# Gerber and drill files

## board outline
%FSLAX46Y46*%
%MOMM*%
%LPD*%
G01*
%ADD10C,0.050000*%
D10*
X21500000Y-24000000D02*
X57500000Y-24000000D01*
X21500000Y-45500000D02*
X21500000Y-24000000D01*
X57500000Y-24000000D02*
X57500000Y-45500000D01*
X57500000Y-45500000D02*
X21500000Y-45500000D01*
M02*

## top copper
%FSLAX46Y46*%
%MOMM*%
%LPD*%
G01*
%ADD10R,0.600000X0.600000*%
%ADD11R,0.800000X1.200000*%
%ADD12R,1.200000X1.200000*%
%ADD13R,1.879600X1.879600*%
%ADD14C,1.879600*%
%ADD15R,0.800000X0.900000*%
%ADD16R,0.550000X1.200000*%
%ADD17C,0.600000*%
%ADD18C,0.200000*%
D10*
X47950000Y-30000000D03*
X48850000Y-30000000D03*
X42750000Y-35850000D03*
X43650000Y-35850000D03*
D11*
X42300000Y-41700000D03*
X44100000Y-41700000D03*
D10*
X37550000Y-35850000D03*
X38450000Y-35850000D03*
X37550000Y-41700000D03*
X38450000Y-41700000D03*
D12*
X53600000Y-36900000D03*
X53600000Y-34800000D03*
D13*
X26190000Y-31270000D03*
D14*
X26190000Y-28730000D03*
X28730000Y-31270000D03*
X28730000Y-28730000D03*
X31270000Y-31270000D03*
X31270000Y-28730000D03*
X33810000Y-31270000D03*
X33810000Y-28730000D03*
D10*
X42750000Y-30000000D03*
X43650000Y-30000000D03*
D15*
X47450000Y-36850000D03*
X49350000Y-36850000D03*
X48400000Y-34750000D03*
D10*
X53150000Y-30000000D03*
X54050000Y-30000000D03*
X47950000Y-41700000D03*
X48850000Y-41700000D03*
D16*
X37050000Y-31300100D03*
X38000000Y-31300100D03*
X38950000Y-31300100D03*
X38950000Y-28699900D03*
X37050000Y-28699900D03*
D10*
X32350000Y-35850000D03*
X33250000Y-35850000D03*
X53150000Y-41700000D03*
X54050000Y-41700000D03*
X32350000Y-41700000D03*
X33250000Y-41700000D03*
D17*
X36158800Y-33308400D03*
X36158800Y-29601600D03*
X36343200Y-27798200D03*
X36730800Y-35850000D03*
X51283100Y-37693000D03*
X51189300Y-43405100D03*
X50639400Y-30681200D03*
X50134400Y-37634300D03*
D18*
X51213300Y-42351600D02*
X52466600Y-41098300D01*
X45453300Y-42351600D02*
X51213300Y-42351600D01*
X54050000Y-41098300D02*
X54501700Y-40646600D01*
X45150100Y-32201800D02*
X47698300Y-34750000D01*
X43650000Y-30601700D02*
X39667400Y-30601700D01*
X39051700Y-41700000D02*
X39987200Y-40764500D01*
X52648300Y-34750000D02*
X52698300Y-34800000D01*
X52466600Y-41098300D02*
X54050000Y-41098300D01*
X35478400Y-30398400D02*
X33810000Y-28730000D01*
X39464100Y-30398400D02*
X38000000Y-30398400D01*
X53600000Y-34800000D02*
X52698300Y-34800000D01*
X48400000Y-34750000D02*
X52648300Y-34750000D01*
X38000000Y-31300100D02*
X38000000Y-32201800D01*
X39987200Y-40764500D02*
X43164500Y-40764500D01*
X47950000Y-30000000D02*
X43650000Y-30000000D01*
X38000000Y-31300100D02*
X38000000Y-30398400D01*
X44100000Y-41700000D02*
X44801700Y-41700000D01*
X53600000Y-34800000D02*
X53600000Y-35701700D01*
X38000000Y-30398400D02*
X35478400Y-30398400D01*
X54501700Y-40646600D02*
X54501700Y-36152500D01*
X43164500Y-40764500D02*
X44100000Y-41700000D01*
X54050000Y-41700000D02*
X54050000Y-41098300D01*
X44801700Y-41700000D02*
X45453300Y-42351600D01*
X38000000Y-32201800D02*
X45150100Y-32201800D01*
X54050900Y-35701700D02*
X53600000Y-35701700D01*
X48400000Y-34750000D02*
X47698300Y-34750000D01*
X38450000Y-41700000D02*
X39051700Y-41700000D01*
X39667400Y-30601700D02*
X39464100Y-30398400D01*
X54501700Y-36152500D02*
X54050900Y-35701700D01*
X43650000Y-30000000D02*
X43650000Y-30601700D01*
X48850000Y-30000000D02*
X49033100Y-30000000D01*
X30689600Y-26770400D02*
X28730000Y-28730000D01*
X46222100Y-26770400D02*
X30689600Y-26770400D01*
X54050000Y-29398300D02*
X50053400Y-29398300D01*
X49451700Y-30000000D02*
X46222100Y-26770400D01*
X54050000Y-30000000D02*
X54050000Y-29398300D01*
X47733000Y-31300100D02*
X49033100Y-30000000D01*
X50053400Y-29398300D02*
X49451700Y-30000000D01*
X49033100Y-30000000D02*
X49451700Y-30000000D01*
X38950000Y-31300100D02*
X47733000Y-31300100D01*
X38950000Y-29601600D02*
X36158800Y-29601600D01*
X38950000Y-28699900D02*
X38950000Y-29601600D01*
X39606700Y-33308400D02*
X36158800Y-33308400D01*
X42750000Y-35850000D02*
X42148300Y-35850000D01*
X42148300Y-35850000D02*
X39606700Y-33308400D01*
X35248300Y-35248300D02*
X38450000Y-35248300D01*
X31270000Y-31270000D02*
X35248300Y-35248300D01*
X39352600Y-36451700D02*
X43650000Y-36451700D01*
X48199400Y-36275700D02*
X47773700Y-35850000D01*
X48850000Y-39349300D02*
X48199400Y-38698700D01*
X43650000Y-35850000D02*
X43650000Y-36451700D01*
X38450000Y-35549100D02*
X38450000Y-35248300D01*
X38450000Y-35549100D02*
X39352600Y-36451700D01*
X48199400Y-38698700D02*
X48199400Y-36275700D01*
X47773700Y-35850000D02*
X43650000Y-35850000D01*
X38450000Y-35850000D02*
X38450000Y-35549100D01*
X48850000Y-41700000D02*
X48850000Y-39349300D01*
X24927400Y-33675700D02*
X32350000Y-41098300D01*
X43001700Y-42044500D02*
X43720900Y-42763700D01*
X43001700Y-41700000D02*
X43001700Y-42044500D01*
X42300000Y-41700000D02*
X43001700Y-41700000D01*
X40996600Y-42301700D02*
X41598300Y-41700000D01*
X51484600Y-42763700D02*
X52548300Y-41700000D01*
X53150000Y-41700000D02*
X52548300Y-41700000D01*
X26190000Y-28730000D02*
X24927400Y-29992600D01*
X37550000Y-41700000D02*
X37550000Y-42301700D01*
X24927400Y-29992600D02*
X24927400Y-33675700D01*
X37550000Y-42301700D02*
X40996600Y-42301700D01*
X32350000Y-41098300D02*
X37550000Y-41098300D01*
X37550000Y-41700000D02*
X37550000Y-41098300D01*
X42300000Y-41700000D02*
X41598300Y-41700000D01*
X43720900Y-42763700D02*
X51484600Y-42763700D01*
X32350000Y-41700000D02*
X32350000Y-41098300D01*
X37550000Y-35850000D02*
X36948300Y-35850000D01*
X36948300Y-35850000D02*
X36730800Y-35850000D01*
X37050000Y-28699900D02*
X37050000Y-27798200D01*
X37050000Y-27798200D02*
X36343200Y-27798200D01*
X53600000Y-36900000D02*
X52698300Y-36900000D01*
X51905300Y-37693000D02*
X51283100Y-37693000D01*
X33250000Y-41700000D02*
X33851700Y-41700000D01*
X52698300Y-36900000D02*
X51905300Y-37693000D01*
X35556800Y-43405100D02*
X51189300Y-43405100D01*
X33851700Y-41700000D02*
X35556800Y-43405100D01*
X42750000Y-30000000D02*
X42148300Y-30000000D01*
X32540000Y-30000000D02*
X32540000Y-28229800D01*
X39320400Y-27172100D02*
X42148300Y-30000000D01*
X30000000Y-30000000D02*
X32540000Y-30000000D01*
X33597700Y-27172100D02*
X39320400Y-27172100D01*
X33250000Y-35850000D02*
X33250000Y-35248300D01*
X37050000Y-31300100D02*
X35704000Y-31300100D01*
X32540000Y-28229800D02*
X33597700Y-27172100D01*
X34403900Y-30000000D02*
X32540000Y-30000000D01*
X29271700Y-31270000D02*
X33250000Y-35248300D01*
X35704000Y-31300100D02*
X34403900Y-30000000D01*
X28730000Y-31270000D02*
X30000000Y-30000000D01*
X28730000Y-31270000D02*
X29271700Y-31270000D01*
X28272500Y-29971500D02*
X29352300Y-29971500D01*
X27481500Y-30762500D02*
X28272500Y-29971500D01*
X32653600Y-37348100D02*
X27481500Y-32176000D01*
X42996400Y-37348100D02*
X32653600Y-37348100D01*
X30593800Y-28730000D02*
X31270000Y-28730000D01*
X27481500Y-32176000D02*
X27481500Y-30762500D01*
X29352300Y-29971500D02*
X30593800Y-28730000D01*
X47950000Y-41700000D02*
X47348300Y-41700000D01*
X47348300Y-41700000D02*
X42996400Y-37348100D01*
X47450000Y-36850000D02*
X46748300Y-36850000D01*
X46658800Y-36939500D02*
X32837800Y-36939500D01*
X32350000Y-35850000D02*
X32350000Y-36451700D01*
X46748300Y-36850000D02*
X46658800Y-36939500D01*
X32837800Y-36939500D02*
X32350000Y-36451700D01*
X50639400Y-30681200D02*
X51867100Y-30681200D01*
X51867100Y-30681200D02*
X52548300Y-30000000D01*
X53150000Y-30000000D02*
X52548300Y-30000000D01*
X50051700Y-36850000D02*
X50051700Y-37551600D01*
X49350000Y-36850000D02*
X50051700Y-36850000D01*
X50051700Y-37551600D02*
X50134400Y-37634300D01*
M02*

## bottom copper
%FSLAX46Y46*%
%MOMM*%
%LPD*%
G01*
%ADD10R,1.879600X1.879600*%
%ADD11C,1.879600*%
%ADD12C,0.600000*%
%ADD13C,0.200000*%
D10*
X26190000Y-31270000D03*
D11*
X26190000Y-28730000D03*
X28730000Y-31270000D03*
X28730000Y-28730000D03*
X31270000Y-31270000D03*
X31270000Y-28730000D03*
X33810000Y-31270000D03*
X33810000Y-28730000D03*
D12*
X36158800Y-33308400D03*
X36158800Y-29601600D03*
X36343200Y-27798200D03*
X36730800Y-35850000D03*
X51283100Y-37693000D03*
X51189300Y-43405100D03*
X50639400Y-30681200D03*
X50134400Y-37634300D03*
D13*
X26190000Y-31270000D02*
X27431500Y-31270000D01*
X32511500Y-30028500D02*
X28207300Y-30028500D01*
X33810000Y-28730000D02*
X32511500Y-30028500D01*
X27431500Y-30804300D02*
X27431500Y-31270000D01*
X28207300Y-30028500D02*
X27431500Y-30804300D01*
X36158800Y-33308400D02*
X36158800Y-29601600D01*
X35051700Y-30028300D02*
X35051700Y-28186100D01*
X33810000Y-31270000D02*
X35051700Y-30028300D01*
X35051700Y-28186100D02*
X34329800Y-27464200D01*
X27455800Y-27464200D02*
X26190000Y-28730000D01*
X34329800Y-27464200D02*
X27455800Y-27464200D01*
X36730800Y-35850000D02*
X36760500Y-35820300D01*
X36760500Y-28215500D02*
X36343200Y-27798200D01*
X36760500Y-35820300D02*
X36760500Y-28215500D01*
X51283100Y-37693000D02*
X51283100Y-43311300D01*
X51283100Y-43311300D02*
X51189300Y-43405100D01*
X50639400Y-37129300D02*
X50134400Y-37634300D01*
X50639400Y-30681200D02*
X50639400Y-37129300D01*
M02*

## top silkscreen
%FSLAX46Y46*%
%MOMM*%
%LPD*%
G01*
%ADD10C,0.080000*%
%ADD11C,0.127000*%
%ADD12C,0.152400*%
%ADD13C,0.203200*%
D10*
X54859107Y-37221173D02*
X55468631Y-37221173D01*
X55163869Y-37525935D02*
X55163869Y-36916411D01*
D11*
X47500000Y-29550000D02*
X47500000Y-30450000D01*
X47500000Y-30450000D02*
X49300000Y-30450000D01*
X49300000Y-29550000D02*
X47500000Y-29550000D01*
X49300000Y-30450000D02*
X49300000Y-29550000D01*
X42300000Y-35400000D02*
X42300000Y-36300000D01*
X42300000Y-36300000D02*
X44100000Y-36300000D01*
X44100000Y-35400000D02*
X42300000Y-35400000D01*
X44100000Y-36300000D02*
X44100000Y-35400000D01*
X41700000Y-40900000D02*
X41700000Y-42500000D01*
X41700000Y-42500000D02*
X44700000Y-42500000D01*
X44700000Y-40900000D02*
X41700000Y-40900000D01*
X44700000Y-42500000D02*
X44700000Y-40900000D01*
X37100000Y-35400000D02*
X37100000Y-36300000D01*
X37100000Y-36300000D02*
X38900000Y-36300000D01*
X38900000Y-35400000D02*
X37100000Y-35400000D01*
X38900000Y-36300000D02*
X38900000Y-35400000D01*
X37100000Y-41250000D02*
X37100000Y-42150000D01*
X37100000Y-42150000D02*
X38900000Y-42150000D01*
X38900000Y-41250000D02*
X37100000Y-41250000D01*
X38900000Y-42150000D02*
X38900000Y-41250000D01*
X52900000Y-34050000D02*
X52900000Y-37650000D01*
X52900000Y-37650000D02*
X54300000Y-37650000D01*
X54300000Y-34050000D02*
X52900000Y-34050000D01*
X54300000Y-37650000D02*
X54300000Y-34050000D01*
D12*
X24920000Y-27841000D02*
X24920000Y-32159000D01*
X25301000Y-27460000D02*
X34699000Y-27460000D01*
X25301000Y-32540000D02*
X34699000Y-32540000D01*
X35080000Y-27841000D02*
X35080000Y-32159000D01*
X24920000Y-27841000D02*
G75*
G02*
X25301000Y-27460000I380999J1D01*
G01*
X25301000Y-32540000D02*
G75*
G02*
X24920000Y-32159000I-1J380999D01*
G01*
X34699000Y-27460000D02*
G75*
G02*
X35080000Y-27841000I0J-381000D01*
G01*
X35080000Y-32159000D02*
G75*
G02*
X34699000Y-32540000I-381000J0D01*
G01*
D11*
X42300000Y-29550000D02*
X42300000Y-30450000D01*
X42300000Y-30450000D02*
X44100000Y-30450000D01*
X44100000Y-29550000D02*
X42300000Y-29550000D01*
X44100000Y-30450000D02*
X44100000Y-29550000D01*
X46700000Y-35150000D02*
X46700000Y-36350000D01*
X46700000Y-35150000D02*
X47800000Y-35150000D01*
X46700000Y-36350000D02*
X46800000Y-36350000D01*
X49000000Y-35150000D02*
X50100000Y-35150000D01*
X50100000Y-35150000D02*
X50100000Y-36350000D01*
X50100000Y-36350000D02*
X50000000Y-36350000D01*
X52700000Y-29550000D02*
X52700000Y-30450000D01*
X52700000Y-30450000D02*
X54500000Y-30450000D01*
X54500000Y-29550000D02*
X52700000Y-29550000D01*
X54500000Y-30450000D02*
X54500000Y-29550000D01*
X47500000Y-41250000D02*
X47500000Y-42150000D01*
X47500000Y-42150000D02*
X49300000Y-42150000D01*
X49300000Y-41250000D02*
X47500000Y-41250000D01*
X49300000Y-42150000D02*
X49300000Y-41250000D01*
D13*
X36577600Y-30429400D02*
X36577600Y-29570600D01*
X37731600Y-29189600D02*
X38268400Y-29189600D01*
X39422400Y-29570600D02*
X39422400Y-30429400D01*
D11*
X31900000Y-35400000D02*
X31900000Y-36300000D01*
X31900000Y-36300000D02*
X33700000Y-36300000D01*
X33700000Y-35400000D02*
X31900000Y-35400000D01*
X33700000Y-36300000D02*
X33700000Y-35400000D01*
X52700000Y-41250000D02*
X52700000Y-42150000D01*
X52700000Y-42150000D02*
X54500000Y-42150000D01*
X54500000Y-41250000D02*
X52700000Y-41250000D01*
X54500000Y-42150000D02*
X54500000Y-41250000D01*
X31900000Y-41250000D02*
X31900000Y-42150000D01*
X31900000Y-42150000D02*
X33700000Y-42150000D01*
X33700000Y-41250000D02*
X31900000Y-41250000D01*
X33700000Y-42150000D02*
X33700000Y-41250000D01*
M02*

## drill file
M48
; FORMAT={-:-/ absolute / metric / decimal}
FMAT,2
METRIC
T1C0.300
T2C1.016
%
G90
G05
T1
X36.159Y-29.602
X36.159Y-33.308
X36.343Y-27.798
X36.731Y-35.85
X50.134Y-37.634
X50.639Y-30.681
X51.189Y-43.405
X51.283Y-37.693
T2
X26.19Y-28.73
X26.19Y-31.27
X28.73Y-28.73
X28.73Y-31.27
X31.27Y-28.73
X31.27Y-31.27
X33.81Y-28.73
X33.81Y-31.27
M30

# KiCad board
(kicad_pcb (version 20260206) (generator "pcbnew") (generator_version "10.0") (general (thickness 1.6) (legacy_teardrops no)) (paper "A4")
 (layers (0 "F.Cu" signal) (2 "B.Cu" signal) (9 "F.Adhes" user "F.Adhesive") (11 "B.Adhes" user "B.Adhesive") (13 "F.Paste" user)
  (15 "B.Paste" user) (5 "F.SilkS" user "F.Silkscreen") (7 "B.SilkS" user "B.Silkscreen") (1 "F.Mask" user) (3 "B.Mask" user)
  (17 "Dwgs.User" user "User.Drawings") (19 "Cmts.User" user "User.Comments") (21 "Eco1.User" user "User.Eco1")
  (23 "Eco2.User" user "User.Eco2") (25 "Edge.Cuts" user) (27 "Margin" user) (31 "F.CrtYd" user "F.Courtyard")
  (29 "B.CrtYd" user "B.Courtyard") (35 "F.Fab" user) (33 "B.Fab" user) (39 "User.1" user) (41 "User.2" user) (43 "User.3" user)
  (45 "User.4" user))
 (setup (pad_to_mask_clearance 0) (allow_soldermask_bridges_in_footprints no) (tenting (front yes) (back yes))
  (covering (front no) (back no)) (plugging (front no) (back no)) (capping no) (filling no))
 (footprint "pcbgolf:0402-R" (layer "F.Cu") (at 48.4 30)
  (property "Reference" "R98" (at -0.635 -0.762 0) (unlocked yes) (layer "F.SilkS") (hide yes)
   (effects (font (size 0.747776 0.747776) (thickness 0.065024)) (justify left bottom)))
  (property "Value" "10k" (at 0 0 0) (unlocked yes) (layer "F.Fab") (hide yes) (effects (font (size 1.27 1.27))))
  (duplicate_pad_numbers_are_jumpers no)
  (fp_line (start -0.9 -0.45) (end -0.9 0.45) (stroke (width 0.127) (type solid)) (layer "F.SilkS"))
  (fp_line (start -0.9 0.45) (end 0.9 0.45) (stroke (width 0.127) (type solid)) (layer "F.SilkS"))
  (fp_line (start 0.9 -0.45) (end -0.9 -0.45) (stroke (width 0.127) (type solid)) (layer "F.SilkS"))
  (fp_line (start 0.9 0.45) (end 0.9 -0.45) (stroke (width 0.127) (type solid)) (layer "F.SilkS"))
  (pad "1" smd rect (at -0.45 0) (size 0.6 0.6) (layers "F.Cu" "F.Mask" "F.Paste") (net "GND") (solder_mask_margin 0.0508)
   (solder_paste_margin 0) (thermal_bridge_angle 0))
  (pad "2" smd rect (at 0.45 0) (size 0.6 0.6) (layers "F.Cu" "F.Mask" "F.Paste") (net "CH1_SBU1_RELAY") (solder_mask_margin 0.0508)
   (solder_paste_margin 0) (thermal_bridge_angle 0)))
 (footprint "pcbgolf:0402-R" (layer "F.Cu") (at 43.2 35.85)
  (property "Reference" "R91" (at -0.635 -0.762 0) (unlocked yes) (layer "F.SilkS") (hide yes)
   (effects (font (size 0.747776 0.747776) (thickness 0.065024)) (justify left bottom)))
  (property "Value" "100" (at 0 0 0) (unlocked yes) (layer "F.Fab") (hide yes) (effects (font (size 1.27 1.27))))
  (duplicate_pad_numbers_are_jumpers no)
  (fp_line (start -0.9 -0.45) (end -0.9 0.45) (stroke (width 0.127) (type solid)) (layer "F.SilkS"))
  (fp_line (start -0.9 0.45) (end 0.9 0.45) (stroke (width 0.127) (type solid)) (layer "F.SilkS"))
  (fp_line (start 0.9 -0.45) (end -0.9 -0.45) (stroke (width 0.127) (type solid)) (layer "F.SilkS"))
  (fp_line (start 0.9 0.45) (end 0.9 -0.45) (stroke (width 0.127) (type solid)) (layer "F.SilkS"))
  (pad "1" smd rect (at -0.45 0) (size 0.6 0.6) (layers "F.Cu" "F.Mask" "F.Paste") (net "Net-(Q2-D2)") (solder_mask_margin 0.0508)
   (solder_paste_margin 0) (thermal_bridge_angle 0))
  (pad "2" smd rect (at 0.45 0) (size 0.6 0.6) (layers "F.Cu" "F.Mask" "F.Paste") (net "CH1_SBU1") (solder_mask_margin 0.0508)
   (solder_paste_margin 0) (thermal_bridge_angle 0)))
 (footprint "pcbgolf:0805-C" (layer "F.Cu") (at 43.2 41.7)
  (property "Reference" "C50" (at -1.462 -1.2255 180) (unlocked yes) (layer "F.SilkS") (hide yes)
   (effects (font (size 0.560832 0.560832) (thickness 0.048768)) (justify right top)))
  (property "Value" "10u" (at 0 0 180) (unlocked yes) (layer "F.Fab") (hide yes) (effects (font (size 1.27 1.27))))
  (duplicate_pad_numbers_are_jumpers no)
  (fp_line (start -1.5 -0.8) (end -1.5 0.8) (stroke (width 0.127) (type solid)) (layer "F.SilkS"))
  (fp_line (start -1.5 0.8) (end 1.5 0.8) (stroke (width 0.127) (type solid)) (layer "F.SilkS"))
  (fp_line (start 1.5 -0.8) (end -1.5 -0.8) (stroke (width 0.127) (type solid)) (layer "F.SilkS"))
  (fp_line (start 1.5 0.8) (end 1.5 -0.8) (stroke (width 0.127) (type solid)) (layer "F.SilkS"))
  (pad "1" smd rect (at -0.9 0) (size 0.8 1.2) (layers "F.Cu" "F.Mask" "F.Paste") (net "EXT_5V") (solder_mask_margin 0.0508)
   (solder_paste_margin 0) (thermal_bridge_angle 0))
  (pad "2" smd rect (at 0.9 0) (size 0.8 1.2) (layers "F.Cu" "F.Mask" "F.Paste") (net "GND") (solder_mask_margin 0.0508)
   (solder_paste_margin 0) (thermal_bridge_angle 0)))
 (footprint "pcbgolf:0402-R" (layer "F.Cu") (at 38 35.85)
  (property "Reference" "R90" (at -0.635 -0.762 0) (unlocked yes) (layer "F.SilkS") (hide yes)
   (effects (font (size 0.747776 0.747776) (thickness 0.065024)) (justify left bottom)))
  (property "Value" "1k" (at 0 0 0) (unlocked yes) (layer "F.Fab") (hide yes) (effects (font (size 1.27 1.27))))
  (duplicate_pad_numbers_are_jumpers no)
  (fp_line (start -0.9 -0.45) (end -0.9 0.45) (stroke (width 0.127) (type solid)) (layer "F.SilkS"))
  (fp_line (start -0.9 0.45) (end 0.9 0.45) (stroke (width 0.127) (type solid)) (layer "F.SilkS"))
  (fp_line (start 0.9 -0.45) (end -0.9 -0.45) (stroke (width 0.127) (type solid)) (layer "F.SilkS"))
  (fp_line (start 0.9 0.45) (end 0.9 -0.45) (stroke (width 0.127) (type solid)) (layer "F.SilkS"))
  (pad "1" smd rect (at -0.45 0) (size 0.6 0.6) (layers "F.Cu" "F.Mask" "F.Paste") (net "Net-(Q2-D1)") (solder_mask_margin 0.0508)
   (solder_paste_margin 0) (thermal_bridge_angle 0))
  (pad "2" smd rect (at 0.45 0) (size 0.6 0.6) (layers "F.Cu" "F.Mask" "F.Paste") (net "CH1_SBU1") (solder_mask_margin 0.0508)
   (solder_paste_margin 0) (thermal_bridge_angle 0)))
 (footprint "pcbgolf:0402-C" (layer "F.Cu") (at 38 41.7)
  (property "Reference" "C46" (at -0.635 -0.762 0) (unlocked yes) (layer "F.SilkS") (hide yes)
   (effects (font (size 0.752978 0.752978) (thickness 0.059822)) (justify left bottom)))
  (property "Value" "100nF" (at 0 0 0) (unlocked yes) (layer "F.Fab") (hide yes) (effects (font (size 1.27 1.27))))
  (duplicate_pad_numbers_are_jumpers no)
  (fp_line (start -0.9 -0.45) (end -0.9 0.45) (stroke (width 0.127) (type solid)) (layer "F.SilkS"))
  (fp_line (start -0.9 0.45) (end 0.9 0.45) (stroke (width 0.127) (type solid)) (layer "F.SilkS"))
  (fp_line (start 0.9 -0.45) (end -0.9 -0.45) (stroke (width 0.127) (type solid)) (layer "F.SilkS"))
  (fp_line (start 0.9 0.45) (end 0.9 -0.45) (stroke (width 0.127) (type solid)) (layer "F.SilkS"))
  (pad "1" smd rect (at -0.45 0) (size 0.6 0.6) (layers "F.Cu" "F.Mask" "F.Paste") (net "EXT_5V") (solder_mask_margin 0.0508)
   (solder_paste_margin 0) (thermal_bridge_angle 0))
  (pad "2" smd rect (at 0.45 0) (size 0.6 0.6) (layers "F.Cu" "F.Mask" "F.Paste") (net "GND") (solder_mask_margin 0.0508)
   (solder_paste_margin 0) (thermal_bridge_angle 0)))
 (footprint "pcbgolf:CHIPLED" (layer "F.Cu") (at 53.6 35.85)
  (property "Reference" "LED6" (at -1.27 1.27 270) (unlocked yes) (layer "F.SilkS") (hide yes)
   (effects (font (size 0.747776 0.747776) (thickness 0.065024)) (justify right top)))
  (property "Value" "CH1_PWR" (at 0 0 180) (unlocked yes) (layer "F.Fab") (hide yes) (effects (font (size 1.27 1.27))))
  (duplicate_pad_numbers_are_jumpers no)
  (fp_line (start -0.7 -1.8) (end -0.7 1.8) (stroke (width 0.127) (type solid)) (layer "F.SilkS"))
  (fp_line (start -0.7 1.8) (end 0.7 1.8) (stroke (width 0.127) (type solid)) (layer "F.SilkS"))
  (fp_line (start 0.7 -1.8) (end -0.7 -1.8) (stroke (width 0.127) (type solid)) (layer "F.SilkS"))
  (fp_line (start 0.7 1.8) (end 0.7 -1.8) (stroke (width 0.127) (type solid)) (layer "F.SilkS"))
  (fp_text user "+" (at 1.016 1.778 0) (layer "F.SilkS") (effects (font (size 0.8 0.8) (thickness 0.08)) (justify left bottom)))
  (pad "A" smd rect (at 0 1.05) (size 1.2 1.2) (layers "F.Cu" "F.Mask" "F.Paste") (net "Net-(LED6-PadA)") (solder_mask_margin 0.0508)
   (solder_paste_margin 0) (thermal_bridge_angle 0))
  (pad "C" smd rect (at 0 -1.05) (size 1.2 1.2) (layers "F.Cu" "F.Mask" "F.Paste") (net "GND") (solder_mask_margin 0.0508)
   (solder_paste_margin 0) (thermal_bridge_angle 0)))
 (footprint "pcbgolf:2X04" (layer "F.Cu") (at 30 30)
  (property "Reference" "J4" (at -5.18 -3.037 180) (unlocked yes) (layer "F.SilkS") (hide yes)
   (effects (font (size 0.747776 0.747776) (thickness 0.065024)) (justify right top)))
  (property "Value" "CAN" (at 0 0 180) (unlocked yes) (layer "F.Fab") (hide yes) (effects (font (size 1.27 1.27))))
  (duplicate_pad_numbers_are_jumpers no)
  (fp_line (start -5.08 -2.159) (end -5.08 2.159) (stroke (width 0.1524) (type solid)) (layer "F.SilkS"))
  (fp_line (start -4.699 -2.54) (end 4.699 -2.54) (stroke (width 0.1524) (type solid)) (layer "F.SilkS"))
  (fp_line (start -4.699 2.54) (end 4.699 2.54) (stroke (width 0.1524) (type solid)) (layer "F.SilkS"))
  (fp_line (start 5.08 -2.159) (end 5.08 2.159) (stroke (width 0.1524) (type solid)) (layer "F.SilkS"))
  (fp_arc (start -5.08 -2.159) (mid -4.968408 -2.428408) (end -4.699 -2.54) (stroke (width 0.1524) (type solid)) (layer "F.SilkS"))
  (fp_arc (start -4.699 2.54) (mid -4.968408 2.428408) (end -5.08 2.159) (stroke (width 0.1524) (type solid)) (layer "F.SilkS"))
  (fp_arc (start 4.699 -2.54) (mid 4.968408 -2.428408) (end 5.08 -2.159) (stroke (width 0.1524) (type solid)) (layer "F.SilkS"))
  (fp_arc (start 5.08 2.159) (mid 4.968408 2.428408) (end 4.699 2.54) (stroke (width 0.1524) (type solid)) (layer "F.SilkS"))
  (pad "1" thru_hole rect (at -3.81 1.27 90) (size 1.8796 1.8796) (drill 1.016) (layers "*.Cu" "*.Mask") (remove_unused_layers no)
   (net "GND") (solder_mask_margin 0.0508) (thermal_bridge_angle 0))
  (pad "2" thru_hole circle (at -3.81 -1.27 90) (size 1.8796 1.8796) (drill 1.016) (layers "*.Cu" "*.Mask") (remove_unused_layers no)
   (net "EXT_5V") (solder_mask_margin 0.0508) (thermal_bridge_angle 0))
  (pad "3" thru_hole circle (at -1.27 1.27 90) (size 1.8796 1.8796) (drill 1.016) (layers "*.Cu" "*.Mask") (remove_unused_layers no)
   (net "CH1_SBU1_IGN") (solder_mask_margin 0.0508) (thermal_bridge_angle 0))
  (pad "4" thru_hole circle (at -1.27 -1.27 90) (size 1.8796 1.8796) (drill 1.016) (layers "*.Cu" "*.Mask") (remove_unused_layers no)
   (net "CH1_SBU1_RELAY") (solder_mask_margin 0.0508) (thermal_bridge_angle 0))
  (pad "5" thru_hole circle (at 1.27 1.27 90) (size 1.8796 1.8796) (drill 1.016) (layers "*.Cu" "*.Mask") (remove_unused_layers no)
   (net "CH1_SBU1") (solder_mask_margin 0.0508) (thermal_bridge_angle 0))
  (pad "6" thru_hole circle (at 1.27 -1.27 90) (size 1.8796 1.8796) (drill 1.016) (layers "*.Cu" "*.Mask") (remove_unused_layers no)
   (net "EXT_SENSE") (solder_mask_margin 0.0508) (thermal_bridge_angle 0))
  (pad "7" thru_hole circle (at 3.81 1.27 90) (size 1.8796 1.8796) (drill 1.016) (layers "*.Cu" "*.Mask") (remove_unused_layers no)
   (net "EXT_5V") (solder_mask_margin 0.0508) (thermal_bridge_angle 0))
  (pad "8" thru_hole circle (at 3.81 -1.27 90) (size 1.8796 1.8796) (drill 1.016) (layers "*.Cu" "*.Mask") (remove_unused_layers no)
   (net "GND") (solder_mask_margin 0.0508) (thermal_bridge_angle 0)))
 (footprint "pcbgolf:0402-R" (layer "F.Cu") (at 43.2 30)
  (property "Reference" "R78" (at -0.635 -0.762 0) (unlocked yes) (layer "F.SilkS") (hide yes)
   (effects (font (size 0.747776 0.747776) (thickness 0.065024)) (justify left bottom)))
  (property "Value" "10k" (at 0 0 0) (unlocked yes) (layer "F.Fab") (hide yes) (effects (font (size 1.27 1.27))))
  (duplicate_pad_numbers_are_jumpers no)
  (fp_line (start -0.9 -0.45) (end -0.9 0.45) (stroke (width 0.127) (type solid)) (layer "F.SilkS"))
  (fp_line (start -0.9 0.45) (end 0.9 0.45) (stroke (width 0.127) (type solid)) (layer "F.SilkS"))
  (fp_line (start 0.9 -0.45) (end -0.9 -0.45) (stroke (width 0.127) (type solid)) (layer "F.SilkS"))
  (fp_line (start 0.9 0.45) (end 0.9 -0.45) (stroke (width 0.127) (type solid)) (layer "F.SilkS"))
  (pad "1" smd rect (at -0.45 0) (size 0.6 0.6) (layers "F.Cu" "F.Mask" "F.Paste") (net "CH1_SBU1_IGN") (solder_mask_margin 0.0508)
   (solder_paste_margin 0) (thermal_bridge_angle 0))
  (pad "2" smd rect (at 0.45 0) (size 0.6 0.6) (layers "F.Cu" "F.Mask" "F.Paste") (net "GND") (solder_mask_margin 0.0508)
   (solder_paste_margin 0) (thermal_bridge_angle 0)))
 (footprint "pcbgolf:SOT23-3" (layer "F.Cu") (at 48.4 35.85)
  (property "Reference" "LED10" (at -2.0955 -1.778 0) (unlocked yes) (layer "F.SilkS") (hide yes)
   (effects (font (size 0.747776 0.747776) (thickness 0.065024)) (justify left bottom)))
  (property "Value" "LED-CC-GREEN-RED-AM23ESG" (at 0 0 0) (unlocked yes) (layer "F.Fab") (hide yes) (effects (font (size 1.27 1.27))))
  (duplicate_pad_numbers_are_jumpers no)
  (fp_line (start -1.7 -0.7) (end -1.7 0.5) (stroke (width 0.127) (type solid)) (layer "F.SilkS"))
  (fp_line (start -1.7 -0.7) (end -0.6 -0.7) (stroke (width 0.127) (type solid)) (layer "F.SilkS"))
  (fp_line (start -1.7 0.5) (end -1.6 0.5) (stroke (width 0.127) (type solid)) (layer "F.SilkS"))
  (fp_line (start 0.6 -0.7) (end 1.7 -0.7) (stroke (width 0.127) (type solid)) (layer "F.SilkS"))
  (fp_line (start 1.7 -0.7) (end 1.7 0.5) (stroke (width 0.127) (type solid)) (layer "F.SilkS"))
  (fp_line (start 1.7 0.5) (end 1.6 0.5) (stroke (width 0.127) (type solid)) (layer "F.SilkS"))
  (pad "1" smd rect (at -0.95 1) (size 0.8 0.9) (layers "F.Cu" "F.Mask" "F.Paste") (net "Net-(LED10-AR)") (solder_mask_margin 0.0508)
   (solder_paste_margin 0) (thermal_bridge_angle 0))
  (pad "2" smd rect (at 0.95 1) (size 0.8 0.9) (layers "F.Cu" "F.Mask" "F.Paste") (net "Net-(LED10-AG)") (solder_mask_margin 0.0508)
   (solder_paste_margin 0) (thermal_bridge_angle 0))
  (pad "3" smd rect (at 0 -1.1) (size 0.8 0.9) (layers "F.Cu" "F.Mask" "F.Paste") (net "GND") (solder_mask_margin 0.0508)
   (solder_paste_margin 0) (thermal_bridge_angle 0)))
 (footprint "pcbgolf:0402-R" (layer "F.Cu") (at 53.6 30)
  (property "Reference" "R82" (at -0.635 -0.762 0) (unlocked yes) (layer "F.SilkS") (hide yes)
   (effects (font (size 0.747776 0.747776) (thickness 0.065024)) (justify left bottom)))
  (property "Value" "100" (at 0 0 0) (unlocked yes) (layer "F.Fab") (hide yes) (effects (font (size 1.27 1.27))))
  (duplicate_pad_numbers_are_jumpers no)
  (fp_line (start -0.9 -0.45) (end -0.9 0.45) (stroke (width 0.127) (type solid)) (layer "F.SilkS"))
  (fp_line (start -0.9 0.45) (end 0.9 0.45) (stroke (width 0.127) (type solid)) (layer "F.SilkS"))
  (fp_line (start 0.9 -0.45) (end -0.9 -0.45) (stroke (width 0.127) (type solid)) (layer "F.SilkS"))
  (fp_line (start 0.9 0.45) (end 0.9 -0.45) (stroke (width 0.127) (type solid)) (layer "F.SilkS"))
  (pad "1" smd rect (at -0.45 0) (size 0.6 0.6) (layers "F.Cu" "F.Mask" "F.Paste") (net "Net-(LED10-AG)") (solder_mask_margin 0.0508)
   (solder_paste_margin 0) (thermal_bridge_angle 0))
  (pad "2" smd rect (at 0.45 0) (size 0.6 0.6) (layers "F.Cu" "F.Mask" "F.Paste") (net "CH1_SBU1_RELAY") (solder_mask_margin 0.0508)
   (solder_paste_margin 0) (thermal_bridge_angle 0)))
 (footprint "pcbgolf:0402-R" (layer "F.Cu") (at 48.4 41.7)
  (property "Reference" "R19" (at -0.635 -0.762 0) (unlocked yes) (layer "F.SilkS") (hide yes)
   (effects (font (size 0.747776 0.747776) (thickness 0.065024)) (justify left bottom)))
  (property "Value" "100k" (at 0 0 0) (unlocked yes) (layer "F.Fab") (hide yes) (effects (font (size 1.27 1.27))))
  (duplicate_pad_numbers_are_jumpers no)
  (fp_line (start -0.9 -0.45) (end -0.9 0.45) (stroke (width 0.127) (type solid)) (layer "F.SilkS"))
  (fp_line (start -0.9 0.45) (end 0.9 0.45) (stroke (width 0.127) (type solid)) (layer "F.SilkS"))
  (fp_line (start 0.9 -0.45) (end -0.9 -0.45) (stroke (width 0.127) (type solid)) (layer "F.SilkS"))
  (fp_line (start 0.9 0.45) (end 0.9 -0.45) (stroke (width 0.127) (type solid)) (layer "F.SilkS"))
  (pad "1" smd rect (at -0.45 0) (size 0.6 0.6) (layers "F.Cu" "F.Mask" "F.Paste") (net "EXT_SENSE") (solder_mask_margin 0.0508)
   (solder_paste_margin 0) (thermal_bridge_angle 0))
  (pad "2" smd rect (at 0.45 0) (size 0.6 0.6) (layers "F.Cu" "F.Mask" "F.Paste") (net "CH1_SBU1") (solder_mask_margin 0.0508)
   (solder_paste_margin 0) (thermal_bridge_angle 0)))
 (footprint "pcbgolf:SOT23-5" (layer "F.Cu") (at 38 30)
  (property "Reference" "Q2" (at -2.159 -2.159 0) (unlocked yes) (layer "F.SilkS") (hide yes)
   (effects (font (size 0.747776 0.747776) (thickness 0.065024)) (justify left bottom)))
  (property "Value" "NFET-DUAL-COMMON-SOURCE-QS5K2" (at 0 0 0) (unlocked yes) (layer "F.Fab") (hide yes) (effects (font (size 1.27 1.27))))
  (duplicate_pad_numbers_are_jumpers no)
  (fp_line (start -1.4224 0.4294) (end -1.4224 -0.4294) (stroke (width 0.2032) (type solid)) (layer "F.SilkS"))
  (fp_line (start -0.2684 -0.8104) (end 0.2684 -0.8104) (stroke (width 0.2032) (type solid)) (layer "F.SilkS"))
  (fp_line (start 1.4224 -0.4294) (end 1.4224 0.4294) (stroke (width 0.2032) (type solid)) (layer "F.SilkS"))
  (pad "1" smd rect (at -0.95 1.3001) (size 0.55 1.2) (layers "F.Cu" "F.Mask" "F.Paste") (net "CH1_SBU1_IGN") (solder_mask_margin 0.0508)
   (solder_paste_margin 0) (thermal_bridge_angle 0))
  (pad "2" smd rect (at 0 1.3001) (size 0.55 1.2) (layers "F.Cu" "F.Mask" "F.Paste") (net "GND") (solder_mask_margin 0.0508)
   (solder_paste_margin 0) (thermal_bridge_angle 0))
  (pad "3" smd rect (at 0.95 1.3001) (size 0.55 1.2) (layers "F.Cu" "F.Mask" "F.Paste") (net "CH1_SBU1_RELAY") (solder_mask_margin 0.0508)
   (solder_paste_margin 0) (thermal_bridge_angle 0))
  (pad "4" smd rect (at 0.95 -1.3001) (size 0.55 1.2) (layers "F.Cu" "F.Mask" "F.Paste") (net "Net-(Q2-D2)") (solder_mask_margin 0.0508)
   (solder_paste_margin 0) (thermal_bridge_angle 0))
  (pad "5" smd rect (at -0.95 -1.3001) (size 0.55 1.2) (layers "F.Cu" "F.Mask" "F.Paste") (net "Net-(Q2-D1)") (solder_mask_margin 0.0508)
   (solder_paste_margin 0) (thermal_bridge_angle 0)))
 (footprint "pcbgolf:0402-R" (layer "F.Cu") (at 32.8 35.85)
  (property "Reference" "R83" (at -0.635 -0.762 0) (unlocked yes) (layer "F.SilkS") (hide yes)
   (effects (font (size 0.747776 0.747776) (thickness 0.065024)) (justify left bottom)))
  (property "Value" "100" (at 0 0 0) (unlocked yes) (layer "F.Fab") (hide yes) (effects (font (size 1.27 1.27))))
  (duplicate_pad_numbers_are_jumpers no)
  (fp_line (start -0.9 -0.45) (end -0.9 0.45) (stroke (width 0.127) (type solid)) (layer "F.SilkS"))
  (fp_line (start -0.9 0.45) (end 0.9 0.45) (stroke (width 0.127) (type solid)) (layer "F.SilkS"))
  (fp_line (start 0.9 -0.45) (end -0.9 -0.45) (stroke (width 0.127) (type solid)) (layer "F.SilkS"))
  (fp_line (start 0.9 0.45) (end 0.9 -0.45) (stroke (width 0.127) (type solid)) (layer "F.SilkS"))
  (pad "1" smd rect (at -0.45 0) (size 0.6 0.6) (layers "F.Cu" "F.Mask" "F.Paste") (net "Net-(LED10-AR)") (solder_mask_margin 0.0508)
   (solder_paste_margin 0) (thermal_bridge_angle 0))
  (pad "2" smd rect (at 0.45 0) (size 0.6 0.6) (layers "F.Cu" "F.Mask" "F.Paste") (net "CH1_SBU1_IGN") (solder_mask_margin 0.0508)
   (solder_paste_margin 0) (thermal_bridge_angle 0)))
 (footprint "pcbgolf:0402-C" (layer "F.Cu") (at 53.6 41.7)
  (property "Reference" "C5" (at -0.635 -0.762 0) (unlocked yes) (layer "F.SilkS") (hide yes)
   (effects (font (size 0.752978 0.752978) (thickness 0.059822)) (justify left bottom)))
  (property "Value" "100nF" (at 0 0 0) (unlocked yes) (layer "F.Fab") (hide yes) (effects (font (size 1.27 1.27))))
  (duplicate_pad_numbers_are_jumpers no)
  (fp_line (start -0.9 -0.45) (end -0.9 0.45) (stroke (width 0.127) (type solid)) (layer "F.SilkS"))
  (fp_line (start -0.9 0.45) (end 0.9 0.45) (stroke (width 0.127) (type solid)) (layer "F.SilkS"))
  (fp_line (start 0.9 -0.45) (end -0.9 -0.45) (stroke (width 0.127) (type solid)) (layer "F.SilkS"))
  (fp_line (start 0.9 0.45) (end 0.9 -0.45) (stroke (width 0.127) (type solid)) (layer "F.SilkS"))
  (pad "1" smd rect (at -0.45 0) (size 0.6 0.6) (layers "F.Cu" "F.Mask" "F.Paste") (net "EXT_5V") (solder_mask_margin 0.0508)
   (solder_paste_margin 0) (thermal_bridge_angle 0))
  (pad "2" smd rect (at 0.45 0) (size 0.6 0.6) (layers "F.Cu" "F.Mask" "F.Paste") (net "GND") (solder_mask_margin 0.0508)
   (solder_paste_margin 0) (thermal_bridge_angle 0)))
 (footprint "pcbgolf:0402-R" (layer "F.Cu") (at 32.8 41.7)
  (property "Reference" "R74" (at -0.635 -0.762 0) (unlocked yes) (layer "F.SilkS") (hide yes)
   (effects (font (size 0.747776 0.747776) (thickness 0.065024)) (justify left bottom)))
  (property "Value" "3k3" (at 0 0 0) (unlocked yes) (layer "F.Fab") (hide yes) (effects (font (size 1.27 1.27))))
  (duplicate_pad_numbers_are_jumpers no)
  (fp_line (start -0.9 -0.45) (end -0.9 0.45) (stroke (width 0.127) (type solid)) (layer "F.SilkS"))
  (fp_line (start -0.9 0.45) (end 0.9 0.45) (stroke (width 0.127) (type solid)) (layer "F.SilkS"))
  (fp_line (start 0.9 -0.45) (end -0.9 -0.45) (stroke (width 0.127) (type solid)) (layer "F.SilkS"))
  (fp_line (start 0.9 0.45) (end 0.9 -0.45) (stroke (width 0.127) (type solid)) (layer "F.SilkS"))
  (pad "1" smd rect (at -0.45 0) (size 0.6 0.6) (layers "F.Cu" "F.Mask" "F.Paste") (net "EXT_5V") (solder_mask_margin 0.0508)
   (solder_paste_margin 0) (thermal_bridge_angle 0))
  (pad "2" smd rect (at 0.45 0) (size 0.6 0.6) (layers "F.Cu" "F.Mask" "F.Paste") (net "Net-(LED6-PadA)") (solder_mask_margin 0.0508)
   (solder_paste_margin 0) (thermal_bridge_angle 0)))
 (gr_line (start 21.5 24) (end 57.5 24) (stroke (width 0.05) (type default)) (layer "Edge.Cuts"))
 (gr_line (start 21.5 45.5) (end 21.5 24) (stroke (width 0.05) (type default)) (layer "Edge.Cuts"))
 (gr_line (start 57.5 24) (end 57.5 45.5) (stroke (width 0.05) (type default)) (layer "Edge.Cuts"))
 (gr_line (start 57.5 45.5) (end 21.5 45.5) (stroke (width 0.05) (type default)) (layer "Edge.Cuts"))
 (segment (start 51.2133 42.3516) (end 52.4666 41.0983) (width 0.2) (layer "F.Cu") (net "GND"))
 (segment (start 45.4533 42.3516) (end 51.2133 42.3516) (width 0.2) (layer "F.Cu") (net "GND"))
 (segment (start 54.05 41.0983) (end 54.5017 40.6466) (width 0.2) (layer "F.Cu") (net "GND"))
 (segment (start 45.1501 32.2018) (end 47.6983 34.75) (width 0.2) (layer "F.Cu") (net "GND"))
 (segment (start 43.65 30.6017) (end 39.6674 30.6017) (width 0.2) (layer "F.Cu") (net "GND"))
 (segment (start 39.0517 41.7) (end 39.9872 40.7645) (width 0.2) (layer "F.Cu") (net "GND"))
 (segment (start 52.6483 34.75) (end 52.6983 34.8) (width 0.2) (layer "F.Cu") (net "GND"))
 (segment (start 52.4666 41.0983) (end 54.05 41.0983) (width 0.2) (layer "F.Cu") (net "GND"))
 (segment (start 35.4784 30.3984) (end 33.81 28.73) (width 0.2) (layer "F.Cu") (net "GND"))
 (segment (start 39.4641 30.3984) (end 38 30.3984) (width 0.2) (layer "F.Cu") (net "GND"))
 (segment (start 53.6 34.8) (end 52.6983 34.8) (width 0.2) (layer "F.Cu") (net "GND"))
 (segment (start 48.4 34.75) (end 52.6483 34.75) (width 0.2) (layer "F.Cu") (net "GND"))
 (segment (start 38 31.3001) (end 38 32.2018) (width 0.2) (layer "F.Cu") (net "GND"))
 (segment (start 39.9872 40.7645) (end 43.1645 40.7645) (width 0.2) (layer "F.Cu") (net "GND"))
 (segment (start 47.95 30) (end 43.65 30) (width 0.2) (layer "F.Cu") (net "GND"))
 (segment (start 38 31.3001) (end 38 30.3984) (width 0.2) (layer "F.Cu") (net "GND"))
 (segment (start 44.1 41.7) (end 44.8017 41.7) (width 0.2) (layer "F.Cu") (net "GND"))
 (segment (start 53.6 34.8) (end 53.6 35.7017) (width 0.2) (layer "F.Cu") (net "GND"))
 (segment (start 38 30.3984) (end 35.4784 30.3984) (width 0.2) (layer "F.Cu") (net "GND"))
 (segment (start 54.5017 40.6466) (end 54.5017 36.1525) (width 0.2) (layer "F.Cu") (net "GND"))
 (segment (start 43.1645 40.7645) (end 44.1 41.7) (width 0.2) (layer "F.Cu") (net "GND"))
 (segment (start 54.05 41.7) (end 54.05 41.0983) (width 0.2) (layer "F.Cu") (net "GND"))
 (segment (start 44.8017 41.7) (end 45.4533 42.3516) (width 0.2) (layer "F.Cu") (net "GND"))
 (segment (start 38 32.2018) (end 45.1501 32.2018) (width 0.2) (layer "F.Cu") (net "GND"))
 (segment (start 54.0509 35.7017) (end 53.6 35.7017) (width 0.2) (layer "F.Cu") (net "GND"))
 (segment (start 48.4 34.75) (end 47.6983 34.75) (width 0.2) (layer "F.Cu") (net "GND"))
 (segment (start 38.45 41.7) (end 39.0517 41.7) (width 0.2) (layer "F.Cu") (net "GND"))
 (segment (start 39.6674 30.6017) (end 39.4641 30.3984) (width 0.2) (layer "F.Cu") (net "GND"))
 (segment (start 54.5017 36.1525) (end 54.0509 35.7017) (width 0.2) (layer "F.Cu") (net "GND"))
 (segment (start 43.65 30) (end 43.65 30.6017) (width 0.2) (layer "F.Cu") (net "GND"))
 (segment (start 26.19 31.27) (end 27.4315 31.27) (width 0.2) (layer "B.Cu") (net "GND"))
 (segment (start 32.5115 30.0285) (end 28.2073 30.0285) (width 0.2) (layer "B.Cu") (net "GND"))
 (segment (start 33.81 28.73) (end 32.5115 30.0285) (width 0.2) (layer "B.Cu") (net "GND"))
 (segment (start 27.4315 30.8043) (end 27.4315 31.27) (width 0.2) (layer "B.Cu") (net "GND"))
 (segment (start 28.2073 30.0285) (end 27.4315 30.8043) (width 0.2) (layer "B.Cu") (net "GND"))
 (segment (start 48.85 30) (end 49.0331 30) (width 0.2) (layer "F.Cu") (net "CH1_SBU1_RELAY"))
 (segment (start 30.6896 26.7704) (end 28.73 28.73) (width 0.2) (layer "F.Cu") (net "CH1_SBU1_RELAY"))
 (segment (start 46.2221 26.7704) (end 30.6896 26.7704) (width 0.2) (layer "F.Cu") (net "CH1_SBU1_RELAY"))
 (segment (start 54.05 29.3983) (end 50.0534 29.3983) (width 0.2) (layer "F.Cu") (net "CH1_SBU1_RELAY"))
 (segment (start 49.4517 30) (end 46.2221 26.7704) (width 0.2) (layer "F.Cu") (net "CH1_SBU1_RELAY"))
 (segment (start 54.05 30) (end 54.05 29.3983) (width 0.2) (layer "F.Cu") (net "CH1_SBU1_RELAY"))
 (segment (start 47.733 31.3001) (end 49.0331 30) (width 0.2) (layer "F.Cu") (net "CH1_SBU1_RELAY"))
 (segment (start 50.0534 29.3983) (end 49.4517 30) (width 0.2) (layer "F.Cu") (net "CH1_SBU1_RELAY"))
 (segment (start 49.0331 30) (end 49.4517 30) (width 0.2) (layer "F.Cu") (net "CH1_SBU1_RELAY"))
 (segment (start 38.95 31.3001) (end 47.733 31.3001) (width 0.2) (layer "F.Cu") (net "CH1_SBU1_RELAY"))
 (segment (start 38.95 29.6016) (end 36.1588 29.6016) (width 0.2) (layer "F.Cu") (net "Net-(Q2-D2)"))
 (segment (start 38.95 28.6999) (end 38.95 29.6016) (width 0.2) (layer "F.Cu") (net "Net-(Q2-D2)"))
 (segment (start 39.6067 33.3084) (end 36.1588 33.3084) (width 0.2) (layer "F.Cu") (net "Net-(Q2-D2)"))
 (segment (start 42.75 35.85) (end 42.1483 35.85) (width 0.2) (layer "F.Cu") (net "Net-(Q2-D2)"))
 (segment (start 42.1483 35.85) (end 39.6067 33.3084) (width 0.2) (layer "F.Cu") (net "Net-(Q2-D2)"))
 (via (at 36.1588 33.3084) (size 0.6) (drill 0.3) (layers "F.Cu" "B.Cu") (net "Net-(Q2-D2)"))
 (via (at 36.1588 29.6016) (size 0.6) (drill 0.3) (layers "F.Cu" "B.Cu") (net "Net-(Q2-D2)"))
 (segment (start 36.1588 33.3084) (end 36.1588 29.6016) (width 0.2) (layer "B.Cu") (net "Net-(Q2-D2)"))
 (segment (start 35.2483 35.2483) (end 38.45 35.2483) (width 0.2) (layer "F.Cu") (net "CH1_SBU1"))
 (segment (start 31.27 31.27) (end 35.2483 35.2483) (width 0.2) (layer "F.Cu") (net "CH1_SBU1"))
 (segment (start 39.3526 36.4517) (end 43.65 36.4517) (width 0.2) (layer "F.Cu") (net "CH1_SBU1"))
 (segment (start 48.1994 36.2757) (end 47.7737 35.85) (width 0.2) (layer "F.Cu") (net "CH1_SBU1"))
 (segment (start 48.85 39.3493) (end 48.1994 38.6987) (width 0.2) (layer "F.Cu") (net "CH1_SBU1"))
 (segment (start 43.65 35.85) (end 43.65 36.4517) (width 0.2) (layer "F.Cu") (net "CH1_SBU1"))
 (segment (start 38.45 35.5491) (end 38.45 35.2483) (width 0.2) (layer "F.Cu") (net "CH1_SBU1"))
 (segment (start 38.45 35.5491) (end 39.3526 36.4517) (width 0.2) (layer "F.Cu") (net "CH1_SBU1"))
 (segment (start 48.1994 38.6987) (end 48.1994 36.2757) (width 0.2) (layer "F.Cu") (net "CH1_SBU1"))
 (segment (start 47.7737 35.85) (end 43.65 35.85) (width 0.2) (layer "F.Cu") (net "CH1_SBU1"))
 (segment (start 38.45 35.85) (end 38.45 35.5491) (width 0.2) (layer "F.Cu") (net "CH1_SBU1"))
 (segment (start 48.85 41.7) (end 48.85 39.3493) (width 0.2) (layer "F.Cu") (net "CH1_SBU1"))
 (segment (start 24.9274 33.6757) (end 32.35 41.0983) (width 0.2) (layer "F.Cu") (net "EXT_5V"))
 (segment (start 43.0017 42.0445) (end 43.7209 42.7637) (width 0.2) (layer "F.Cu") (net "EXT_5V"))
 (segment (start 43.0017 41.7) (end 43.0017 42.0445) (width 0.2) (layer "F.Cu") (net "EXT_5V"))
 (segment (start 42.3 41.7) (end 43.0017 41.7) (width 0.2) (layer "F.Cu") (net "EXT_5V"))
 (segment (start 40.9966 42.3017) (end 41.5983 41.7) (width 0.2) (layer "F.Cu") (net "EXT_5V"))
 (segment (start 51.4846 42.7637) (end 52.5483 41.7) (width 0.2) (layer "F.Cu") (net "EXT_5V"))
 (segment (start 53.15 41.7) (end 52.5483 41.7) (width 0.2) (layer "F.Cu") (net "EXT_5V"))
 (segment (start 26.19 28.73) (end 24.9274 29.9926) (width 0.2) (layer "F.Cu") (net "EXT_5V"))
 (segment (start 37.55 41.7) (end 37.55 42.3017) (width 0.2) (layer "F.Cu") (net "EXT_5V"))
 (segment (start 24.9274 29.9926) (end 24.9274 33.6757) (width 0.2) (layer "F.Cu") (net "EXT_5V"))
 (segment (start 37.55 42.3017) (end 40.9966 42.3017) (width 0.2) (layer "F.Cu") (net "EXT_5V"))
 (segment (start 32.35 41.0983) (end 37.55 41.0983) (width 0.2) (layer "F.Cu") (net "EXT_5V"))
 (segment (start 37.55 41.7) (end 37.55 41.0983) (width 0.2) (layer "F.Cu") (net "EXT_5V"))
 (segment (start 42.3 41.7) (end 41.5983 41.7) (width 0.2) (layer "F.Cu") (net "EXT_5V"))
 (segment (start 43.7209 42.7637) (end 51.4846 42.7637) (width 0.2) (layer "F.Cu") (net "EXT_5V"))
 (segment (start 32.35 41.7) (end 32.35 41.0983) (width 0.2) (layer "F.Cu") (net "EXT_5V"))
 (segment (start 35.0517 30.0283) (end 35.0517 28.1861) (width 0.2) (layer "B.Cu") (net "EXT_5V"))
 (segment (start 33.81 31.27) (end 35.0517 30.0283) (width 0.2) (layer "B.Cu") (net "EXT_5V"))
 (segment (start 35.0517 28.1861) (end 34.3298 27.4642) (width 0.2) (layer "B.Cu") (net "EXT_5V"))
 (segment (start 27.4558 27.4642) (end 26.19 28.73) (width 0.2) (layer "B.Cu") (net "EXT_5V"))
 (segment (start 34.3298 27.4642) (end 27.4558 27.4642) (width 0.2) (layer "B.Cu") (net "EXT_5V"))
 (segment (start 37.55 35.85) (end 36.9483 35.85) (width 0.2) (layer "F.Cu") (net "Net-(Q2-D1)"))
 (segment (start 36.9483 35.85) (end 36.7308 35.85) (width 0.2) (layer "F.Cu") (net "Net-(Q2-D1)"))
 (segment (start 37.05 28.6999) (end 37.05 27.7982) (width 0.2) (layer "F.Cu") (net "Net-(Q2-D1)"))
 (segment (start 37.05 27.7982) (end 36.3432 27.7982) (width 0.2) (layer "F.Cu") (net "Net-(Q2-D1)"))
 (via (at 36.3432 27.7982) (size 0.6) (drill 0.3) (layers "F.Cu" "B.Cu") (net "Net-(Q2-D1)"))
 (via (at 36.7308 35.85) (size 0.6) (drill 0.3) (layers "F.Cu" "B.Cu") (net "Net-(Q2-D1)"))
 (segment (start 36.7308 35.85) (end 36.7605 35.8203) (width 0.2) (layer "B.Cu") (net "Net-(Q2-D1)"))
 (segment (start 36.7605 28.2155) (end 36.3432 27.7982) (width 0.2) (layer "B.Cu") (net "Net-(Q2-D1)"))
 (segment (start 36.7605 35.8203) (end 36.7605 28.2155) (width 0.2) (layer "B.Cu") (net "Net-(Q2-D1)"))
 (segment (start 53.6 36.9) (end 52.6983 36.9) (width 0.2) (layer "F.Cu") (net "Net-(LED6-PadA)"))
 (segment (start 51.9053 37.693) (end 51.2831 37.693) (width 0.2) (layer "F.Cu") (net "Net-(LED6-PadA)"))
 (segment (start 33.25 41.7) (end 33.8517 41.7) (width 0.2) (layer "F.Cu") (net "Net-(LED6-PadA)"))
 (segment (start 52.6983 36.9) (end 51.9053 37.693) (width 0.2) (layer "F.Cu") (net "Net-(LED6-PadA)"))
 (segment (start 35.5568 43.4051) (end 51.1893 43.4051) (width 0.2) (layer "F.Cu") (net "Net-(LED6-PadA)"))
 (segment (start 33.8517 41.7) (end 35.5568 43.4051) (width 0.2) (layer "F.Cu") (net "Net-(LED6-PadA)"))
 (via (at 51.2831 37.693) (size 0.6) (drill 0.3) (layers "F.Cu" "B.Cu") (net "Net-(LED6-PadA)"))
 (via (at 51.1893 43.4051) (size 0.6) (drill 0.3) (layers "F.Cu" "B.Cu") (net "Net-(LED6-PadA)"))
 (segment (start 51.2831 37.693) (end 51.2831 43.3113) (width 0.2) (layer "B.Cu") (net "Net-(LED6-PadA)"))
 (segment (start 51.2831 43.3113) (end 51.1893 43.4051) (width 0.2) (layer "B.Cu") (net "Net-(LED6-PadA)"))
 (segment (start 42.75 30) (end 42.1483 30) (width 0.2) (layer "F.Cu") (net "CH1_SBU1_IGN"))
 (segment (start 32.54 30) (end 32.54 28.2298) (width 0.2) (layer "F.Cu") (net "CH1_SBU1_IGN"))
 (segment (start 39.3204 27.1721) (end 42.1483 30) (width 0.2) (layer "F.Cu") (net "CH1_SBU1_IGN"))
 (segment (start 30 30) (end 32.54 30) (width 0.2) (layer "F.Cu") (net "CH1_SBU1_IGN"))
 (segment (start 33.5977 27.1721) (end 39.3204 27.1721) (width 0.2) (layer "F.Cu") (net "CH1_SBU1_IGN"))
 (segment (start 33.25 35.85) (end 33.25 35.2483) (width 0.2) (layer "F.Cu") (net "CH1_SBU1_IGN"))
 (segment (start 37.05 31.3001) (end 35.704 31.3001) (width 0.2) (layer "F.Cu") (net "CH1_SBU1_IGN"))
 (segment (start 32.54 28.2298) (end 33.5977 27.1721) (width 0.2) (layer "F.Cu") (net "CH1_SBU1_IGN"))
 (segment (start 34.4039 30) (end 32.54 30) (width 0.2) (layer "F.Cu") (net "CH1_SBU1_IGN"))
 (segment (start 29.2717 31.27) (end 33.25 35.2483) (width 0.2) (layer "F.Cu") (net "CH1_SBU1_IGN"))
 (segment (start 35.704 31.3001) (end 34.4039 30) (width 0.2) (layer "F.Cu") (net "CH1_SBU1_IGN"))
 (segment (start 28.73 31.27) (end 30 30) (width 0.2) (layer "F.Cu") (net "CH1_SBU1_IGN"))
 (segment (start 28.73 31.27) (end 29.2717 31.27) (width 0.2) (layer "F.Cu") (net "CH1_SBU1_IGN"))
 (segment (start 28.2725 29.9715) (end 29.3523 29.9715) (width 0.2) (layer "F.Cu") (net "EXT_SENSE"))
 (segment (start 27.4815 30.7625) (end 28.2725 29.9715) (width 0.2) (layer "F.Cu") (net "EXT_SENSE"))
 (segment (start 32.6536 37.3481) (end 27.4815 32.176) (width 0.2) (layer "F.Cu") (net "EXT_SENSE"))
 (segment (start 42.9964 37.3481) (end 32.6536 37.3481) (width 0.2) (layer "F.Cu") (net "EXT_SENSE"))
 (segment (start 30.5938 28.73) (end 31.27 28.73) (width 0.2) (layer "F.Cu") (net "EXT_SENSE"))
 (segment (start 27.4815 32.176) (end 27.4815 30.7625) (width 0.2) (layer "F.Cu") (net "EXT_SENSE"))
 (segment (start 29.3523 29.9715) (end 30.5938 28.73) (width 0.2) (layer "F.Cu") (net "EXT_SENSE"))
 (segment (start 47.95 41.7) (end 47.3483 41.7) (width 0.2) (layer "F.Cu") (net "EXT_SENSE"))
 (segment (start 47.3483 41.7) (end 42.9964 37.3481) (width 0.2) (layer "F.Cu") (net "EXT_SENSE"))
 (segment (start 47.45 36.85) (end 46.7483 36.85) (width 0.2) (layer "F.Cu") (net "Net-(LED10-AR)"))
 (segment (start 46.6588 36.9395) (end 32.8378 36.9395) (width 0.2) (layer "F.Cu") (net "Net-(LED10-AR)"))
 (segment (start 32.35 35.85) (end 32.35 36.4517) (width 0.2) (layer "F.Cu") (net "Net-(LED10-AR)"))
 (segment (start 46.7483 36.85) (end 46.6588 36.9395) (width 0.2) (layer "F.Cu") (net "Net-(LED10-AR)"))
 (segment (start 32.8378 36.9395) (end 32.35 36.4517) (width 0.2) (layer "F.Cu") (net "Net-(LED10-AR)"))
 (segment (start 50.6394 30.6812) (end 51.8671 30.6812) (width 0.2) (layer "F.Cu") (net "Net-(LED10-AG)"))
 (segment (start 51.8671 30.6812) (end 52.5483 30) (width 0.2) (layer "F.Cu") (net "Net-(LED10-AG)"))
 (segment (start 53.15 30) (end 52.5483 30) (width 0.2) (layer "F.Cu") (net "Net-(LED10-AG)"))
 (segment (start 50.0517 36.85) (end 50.0517 37.5516) (width 0.2) (layer "F.Cu") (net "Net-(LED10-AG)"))
 (segment (start 49.35 36.85) (end 50.0517 36.85) (width 0.2) (layer "F.Cu") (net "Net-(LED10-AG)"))
 (segment (start 50.0517 37.5516) (end 50.1344 37.6343) (width 0.2) (layer "F.Cu") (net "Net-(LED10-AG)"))
 (via (at 50.6394 30.6812) (size 0.6) (drill 0.3) (layers "F.Cu" "B.Cu") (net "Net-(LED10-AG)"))
 (via (at 50.1344 37.6343) (size 0.6) (drill 0.3) (layers "F.Cu" "B.Cu") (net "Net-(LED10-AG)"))
 (segment (start 50.6394 37.1293) (end 50.1344 37.6343) (width 0.2) (layer "B.Cu") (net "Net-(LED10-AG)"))
 (segment (start 50.6394 30.6812) (end 50.6394 37.1293) (width 0.2) (layer "B.Cu") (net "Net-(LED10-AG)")))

